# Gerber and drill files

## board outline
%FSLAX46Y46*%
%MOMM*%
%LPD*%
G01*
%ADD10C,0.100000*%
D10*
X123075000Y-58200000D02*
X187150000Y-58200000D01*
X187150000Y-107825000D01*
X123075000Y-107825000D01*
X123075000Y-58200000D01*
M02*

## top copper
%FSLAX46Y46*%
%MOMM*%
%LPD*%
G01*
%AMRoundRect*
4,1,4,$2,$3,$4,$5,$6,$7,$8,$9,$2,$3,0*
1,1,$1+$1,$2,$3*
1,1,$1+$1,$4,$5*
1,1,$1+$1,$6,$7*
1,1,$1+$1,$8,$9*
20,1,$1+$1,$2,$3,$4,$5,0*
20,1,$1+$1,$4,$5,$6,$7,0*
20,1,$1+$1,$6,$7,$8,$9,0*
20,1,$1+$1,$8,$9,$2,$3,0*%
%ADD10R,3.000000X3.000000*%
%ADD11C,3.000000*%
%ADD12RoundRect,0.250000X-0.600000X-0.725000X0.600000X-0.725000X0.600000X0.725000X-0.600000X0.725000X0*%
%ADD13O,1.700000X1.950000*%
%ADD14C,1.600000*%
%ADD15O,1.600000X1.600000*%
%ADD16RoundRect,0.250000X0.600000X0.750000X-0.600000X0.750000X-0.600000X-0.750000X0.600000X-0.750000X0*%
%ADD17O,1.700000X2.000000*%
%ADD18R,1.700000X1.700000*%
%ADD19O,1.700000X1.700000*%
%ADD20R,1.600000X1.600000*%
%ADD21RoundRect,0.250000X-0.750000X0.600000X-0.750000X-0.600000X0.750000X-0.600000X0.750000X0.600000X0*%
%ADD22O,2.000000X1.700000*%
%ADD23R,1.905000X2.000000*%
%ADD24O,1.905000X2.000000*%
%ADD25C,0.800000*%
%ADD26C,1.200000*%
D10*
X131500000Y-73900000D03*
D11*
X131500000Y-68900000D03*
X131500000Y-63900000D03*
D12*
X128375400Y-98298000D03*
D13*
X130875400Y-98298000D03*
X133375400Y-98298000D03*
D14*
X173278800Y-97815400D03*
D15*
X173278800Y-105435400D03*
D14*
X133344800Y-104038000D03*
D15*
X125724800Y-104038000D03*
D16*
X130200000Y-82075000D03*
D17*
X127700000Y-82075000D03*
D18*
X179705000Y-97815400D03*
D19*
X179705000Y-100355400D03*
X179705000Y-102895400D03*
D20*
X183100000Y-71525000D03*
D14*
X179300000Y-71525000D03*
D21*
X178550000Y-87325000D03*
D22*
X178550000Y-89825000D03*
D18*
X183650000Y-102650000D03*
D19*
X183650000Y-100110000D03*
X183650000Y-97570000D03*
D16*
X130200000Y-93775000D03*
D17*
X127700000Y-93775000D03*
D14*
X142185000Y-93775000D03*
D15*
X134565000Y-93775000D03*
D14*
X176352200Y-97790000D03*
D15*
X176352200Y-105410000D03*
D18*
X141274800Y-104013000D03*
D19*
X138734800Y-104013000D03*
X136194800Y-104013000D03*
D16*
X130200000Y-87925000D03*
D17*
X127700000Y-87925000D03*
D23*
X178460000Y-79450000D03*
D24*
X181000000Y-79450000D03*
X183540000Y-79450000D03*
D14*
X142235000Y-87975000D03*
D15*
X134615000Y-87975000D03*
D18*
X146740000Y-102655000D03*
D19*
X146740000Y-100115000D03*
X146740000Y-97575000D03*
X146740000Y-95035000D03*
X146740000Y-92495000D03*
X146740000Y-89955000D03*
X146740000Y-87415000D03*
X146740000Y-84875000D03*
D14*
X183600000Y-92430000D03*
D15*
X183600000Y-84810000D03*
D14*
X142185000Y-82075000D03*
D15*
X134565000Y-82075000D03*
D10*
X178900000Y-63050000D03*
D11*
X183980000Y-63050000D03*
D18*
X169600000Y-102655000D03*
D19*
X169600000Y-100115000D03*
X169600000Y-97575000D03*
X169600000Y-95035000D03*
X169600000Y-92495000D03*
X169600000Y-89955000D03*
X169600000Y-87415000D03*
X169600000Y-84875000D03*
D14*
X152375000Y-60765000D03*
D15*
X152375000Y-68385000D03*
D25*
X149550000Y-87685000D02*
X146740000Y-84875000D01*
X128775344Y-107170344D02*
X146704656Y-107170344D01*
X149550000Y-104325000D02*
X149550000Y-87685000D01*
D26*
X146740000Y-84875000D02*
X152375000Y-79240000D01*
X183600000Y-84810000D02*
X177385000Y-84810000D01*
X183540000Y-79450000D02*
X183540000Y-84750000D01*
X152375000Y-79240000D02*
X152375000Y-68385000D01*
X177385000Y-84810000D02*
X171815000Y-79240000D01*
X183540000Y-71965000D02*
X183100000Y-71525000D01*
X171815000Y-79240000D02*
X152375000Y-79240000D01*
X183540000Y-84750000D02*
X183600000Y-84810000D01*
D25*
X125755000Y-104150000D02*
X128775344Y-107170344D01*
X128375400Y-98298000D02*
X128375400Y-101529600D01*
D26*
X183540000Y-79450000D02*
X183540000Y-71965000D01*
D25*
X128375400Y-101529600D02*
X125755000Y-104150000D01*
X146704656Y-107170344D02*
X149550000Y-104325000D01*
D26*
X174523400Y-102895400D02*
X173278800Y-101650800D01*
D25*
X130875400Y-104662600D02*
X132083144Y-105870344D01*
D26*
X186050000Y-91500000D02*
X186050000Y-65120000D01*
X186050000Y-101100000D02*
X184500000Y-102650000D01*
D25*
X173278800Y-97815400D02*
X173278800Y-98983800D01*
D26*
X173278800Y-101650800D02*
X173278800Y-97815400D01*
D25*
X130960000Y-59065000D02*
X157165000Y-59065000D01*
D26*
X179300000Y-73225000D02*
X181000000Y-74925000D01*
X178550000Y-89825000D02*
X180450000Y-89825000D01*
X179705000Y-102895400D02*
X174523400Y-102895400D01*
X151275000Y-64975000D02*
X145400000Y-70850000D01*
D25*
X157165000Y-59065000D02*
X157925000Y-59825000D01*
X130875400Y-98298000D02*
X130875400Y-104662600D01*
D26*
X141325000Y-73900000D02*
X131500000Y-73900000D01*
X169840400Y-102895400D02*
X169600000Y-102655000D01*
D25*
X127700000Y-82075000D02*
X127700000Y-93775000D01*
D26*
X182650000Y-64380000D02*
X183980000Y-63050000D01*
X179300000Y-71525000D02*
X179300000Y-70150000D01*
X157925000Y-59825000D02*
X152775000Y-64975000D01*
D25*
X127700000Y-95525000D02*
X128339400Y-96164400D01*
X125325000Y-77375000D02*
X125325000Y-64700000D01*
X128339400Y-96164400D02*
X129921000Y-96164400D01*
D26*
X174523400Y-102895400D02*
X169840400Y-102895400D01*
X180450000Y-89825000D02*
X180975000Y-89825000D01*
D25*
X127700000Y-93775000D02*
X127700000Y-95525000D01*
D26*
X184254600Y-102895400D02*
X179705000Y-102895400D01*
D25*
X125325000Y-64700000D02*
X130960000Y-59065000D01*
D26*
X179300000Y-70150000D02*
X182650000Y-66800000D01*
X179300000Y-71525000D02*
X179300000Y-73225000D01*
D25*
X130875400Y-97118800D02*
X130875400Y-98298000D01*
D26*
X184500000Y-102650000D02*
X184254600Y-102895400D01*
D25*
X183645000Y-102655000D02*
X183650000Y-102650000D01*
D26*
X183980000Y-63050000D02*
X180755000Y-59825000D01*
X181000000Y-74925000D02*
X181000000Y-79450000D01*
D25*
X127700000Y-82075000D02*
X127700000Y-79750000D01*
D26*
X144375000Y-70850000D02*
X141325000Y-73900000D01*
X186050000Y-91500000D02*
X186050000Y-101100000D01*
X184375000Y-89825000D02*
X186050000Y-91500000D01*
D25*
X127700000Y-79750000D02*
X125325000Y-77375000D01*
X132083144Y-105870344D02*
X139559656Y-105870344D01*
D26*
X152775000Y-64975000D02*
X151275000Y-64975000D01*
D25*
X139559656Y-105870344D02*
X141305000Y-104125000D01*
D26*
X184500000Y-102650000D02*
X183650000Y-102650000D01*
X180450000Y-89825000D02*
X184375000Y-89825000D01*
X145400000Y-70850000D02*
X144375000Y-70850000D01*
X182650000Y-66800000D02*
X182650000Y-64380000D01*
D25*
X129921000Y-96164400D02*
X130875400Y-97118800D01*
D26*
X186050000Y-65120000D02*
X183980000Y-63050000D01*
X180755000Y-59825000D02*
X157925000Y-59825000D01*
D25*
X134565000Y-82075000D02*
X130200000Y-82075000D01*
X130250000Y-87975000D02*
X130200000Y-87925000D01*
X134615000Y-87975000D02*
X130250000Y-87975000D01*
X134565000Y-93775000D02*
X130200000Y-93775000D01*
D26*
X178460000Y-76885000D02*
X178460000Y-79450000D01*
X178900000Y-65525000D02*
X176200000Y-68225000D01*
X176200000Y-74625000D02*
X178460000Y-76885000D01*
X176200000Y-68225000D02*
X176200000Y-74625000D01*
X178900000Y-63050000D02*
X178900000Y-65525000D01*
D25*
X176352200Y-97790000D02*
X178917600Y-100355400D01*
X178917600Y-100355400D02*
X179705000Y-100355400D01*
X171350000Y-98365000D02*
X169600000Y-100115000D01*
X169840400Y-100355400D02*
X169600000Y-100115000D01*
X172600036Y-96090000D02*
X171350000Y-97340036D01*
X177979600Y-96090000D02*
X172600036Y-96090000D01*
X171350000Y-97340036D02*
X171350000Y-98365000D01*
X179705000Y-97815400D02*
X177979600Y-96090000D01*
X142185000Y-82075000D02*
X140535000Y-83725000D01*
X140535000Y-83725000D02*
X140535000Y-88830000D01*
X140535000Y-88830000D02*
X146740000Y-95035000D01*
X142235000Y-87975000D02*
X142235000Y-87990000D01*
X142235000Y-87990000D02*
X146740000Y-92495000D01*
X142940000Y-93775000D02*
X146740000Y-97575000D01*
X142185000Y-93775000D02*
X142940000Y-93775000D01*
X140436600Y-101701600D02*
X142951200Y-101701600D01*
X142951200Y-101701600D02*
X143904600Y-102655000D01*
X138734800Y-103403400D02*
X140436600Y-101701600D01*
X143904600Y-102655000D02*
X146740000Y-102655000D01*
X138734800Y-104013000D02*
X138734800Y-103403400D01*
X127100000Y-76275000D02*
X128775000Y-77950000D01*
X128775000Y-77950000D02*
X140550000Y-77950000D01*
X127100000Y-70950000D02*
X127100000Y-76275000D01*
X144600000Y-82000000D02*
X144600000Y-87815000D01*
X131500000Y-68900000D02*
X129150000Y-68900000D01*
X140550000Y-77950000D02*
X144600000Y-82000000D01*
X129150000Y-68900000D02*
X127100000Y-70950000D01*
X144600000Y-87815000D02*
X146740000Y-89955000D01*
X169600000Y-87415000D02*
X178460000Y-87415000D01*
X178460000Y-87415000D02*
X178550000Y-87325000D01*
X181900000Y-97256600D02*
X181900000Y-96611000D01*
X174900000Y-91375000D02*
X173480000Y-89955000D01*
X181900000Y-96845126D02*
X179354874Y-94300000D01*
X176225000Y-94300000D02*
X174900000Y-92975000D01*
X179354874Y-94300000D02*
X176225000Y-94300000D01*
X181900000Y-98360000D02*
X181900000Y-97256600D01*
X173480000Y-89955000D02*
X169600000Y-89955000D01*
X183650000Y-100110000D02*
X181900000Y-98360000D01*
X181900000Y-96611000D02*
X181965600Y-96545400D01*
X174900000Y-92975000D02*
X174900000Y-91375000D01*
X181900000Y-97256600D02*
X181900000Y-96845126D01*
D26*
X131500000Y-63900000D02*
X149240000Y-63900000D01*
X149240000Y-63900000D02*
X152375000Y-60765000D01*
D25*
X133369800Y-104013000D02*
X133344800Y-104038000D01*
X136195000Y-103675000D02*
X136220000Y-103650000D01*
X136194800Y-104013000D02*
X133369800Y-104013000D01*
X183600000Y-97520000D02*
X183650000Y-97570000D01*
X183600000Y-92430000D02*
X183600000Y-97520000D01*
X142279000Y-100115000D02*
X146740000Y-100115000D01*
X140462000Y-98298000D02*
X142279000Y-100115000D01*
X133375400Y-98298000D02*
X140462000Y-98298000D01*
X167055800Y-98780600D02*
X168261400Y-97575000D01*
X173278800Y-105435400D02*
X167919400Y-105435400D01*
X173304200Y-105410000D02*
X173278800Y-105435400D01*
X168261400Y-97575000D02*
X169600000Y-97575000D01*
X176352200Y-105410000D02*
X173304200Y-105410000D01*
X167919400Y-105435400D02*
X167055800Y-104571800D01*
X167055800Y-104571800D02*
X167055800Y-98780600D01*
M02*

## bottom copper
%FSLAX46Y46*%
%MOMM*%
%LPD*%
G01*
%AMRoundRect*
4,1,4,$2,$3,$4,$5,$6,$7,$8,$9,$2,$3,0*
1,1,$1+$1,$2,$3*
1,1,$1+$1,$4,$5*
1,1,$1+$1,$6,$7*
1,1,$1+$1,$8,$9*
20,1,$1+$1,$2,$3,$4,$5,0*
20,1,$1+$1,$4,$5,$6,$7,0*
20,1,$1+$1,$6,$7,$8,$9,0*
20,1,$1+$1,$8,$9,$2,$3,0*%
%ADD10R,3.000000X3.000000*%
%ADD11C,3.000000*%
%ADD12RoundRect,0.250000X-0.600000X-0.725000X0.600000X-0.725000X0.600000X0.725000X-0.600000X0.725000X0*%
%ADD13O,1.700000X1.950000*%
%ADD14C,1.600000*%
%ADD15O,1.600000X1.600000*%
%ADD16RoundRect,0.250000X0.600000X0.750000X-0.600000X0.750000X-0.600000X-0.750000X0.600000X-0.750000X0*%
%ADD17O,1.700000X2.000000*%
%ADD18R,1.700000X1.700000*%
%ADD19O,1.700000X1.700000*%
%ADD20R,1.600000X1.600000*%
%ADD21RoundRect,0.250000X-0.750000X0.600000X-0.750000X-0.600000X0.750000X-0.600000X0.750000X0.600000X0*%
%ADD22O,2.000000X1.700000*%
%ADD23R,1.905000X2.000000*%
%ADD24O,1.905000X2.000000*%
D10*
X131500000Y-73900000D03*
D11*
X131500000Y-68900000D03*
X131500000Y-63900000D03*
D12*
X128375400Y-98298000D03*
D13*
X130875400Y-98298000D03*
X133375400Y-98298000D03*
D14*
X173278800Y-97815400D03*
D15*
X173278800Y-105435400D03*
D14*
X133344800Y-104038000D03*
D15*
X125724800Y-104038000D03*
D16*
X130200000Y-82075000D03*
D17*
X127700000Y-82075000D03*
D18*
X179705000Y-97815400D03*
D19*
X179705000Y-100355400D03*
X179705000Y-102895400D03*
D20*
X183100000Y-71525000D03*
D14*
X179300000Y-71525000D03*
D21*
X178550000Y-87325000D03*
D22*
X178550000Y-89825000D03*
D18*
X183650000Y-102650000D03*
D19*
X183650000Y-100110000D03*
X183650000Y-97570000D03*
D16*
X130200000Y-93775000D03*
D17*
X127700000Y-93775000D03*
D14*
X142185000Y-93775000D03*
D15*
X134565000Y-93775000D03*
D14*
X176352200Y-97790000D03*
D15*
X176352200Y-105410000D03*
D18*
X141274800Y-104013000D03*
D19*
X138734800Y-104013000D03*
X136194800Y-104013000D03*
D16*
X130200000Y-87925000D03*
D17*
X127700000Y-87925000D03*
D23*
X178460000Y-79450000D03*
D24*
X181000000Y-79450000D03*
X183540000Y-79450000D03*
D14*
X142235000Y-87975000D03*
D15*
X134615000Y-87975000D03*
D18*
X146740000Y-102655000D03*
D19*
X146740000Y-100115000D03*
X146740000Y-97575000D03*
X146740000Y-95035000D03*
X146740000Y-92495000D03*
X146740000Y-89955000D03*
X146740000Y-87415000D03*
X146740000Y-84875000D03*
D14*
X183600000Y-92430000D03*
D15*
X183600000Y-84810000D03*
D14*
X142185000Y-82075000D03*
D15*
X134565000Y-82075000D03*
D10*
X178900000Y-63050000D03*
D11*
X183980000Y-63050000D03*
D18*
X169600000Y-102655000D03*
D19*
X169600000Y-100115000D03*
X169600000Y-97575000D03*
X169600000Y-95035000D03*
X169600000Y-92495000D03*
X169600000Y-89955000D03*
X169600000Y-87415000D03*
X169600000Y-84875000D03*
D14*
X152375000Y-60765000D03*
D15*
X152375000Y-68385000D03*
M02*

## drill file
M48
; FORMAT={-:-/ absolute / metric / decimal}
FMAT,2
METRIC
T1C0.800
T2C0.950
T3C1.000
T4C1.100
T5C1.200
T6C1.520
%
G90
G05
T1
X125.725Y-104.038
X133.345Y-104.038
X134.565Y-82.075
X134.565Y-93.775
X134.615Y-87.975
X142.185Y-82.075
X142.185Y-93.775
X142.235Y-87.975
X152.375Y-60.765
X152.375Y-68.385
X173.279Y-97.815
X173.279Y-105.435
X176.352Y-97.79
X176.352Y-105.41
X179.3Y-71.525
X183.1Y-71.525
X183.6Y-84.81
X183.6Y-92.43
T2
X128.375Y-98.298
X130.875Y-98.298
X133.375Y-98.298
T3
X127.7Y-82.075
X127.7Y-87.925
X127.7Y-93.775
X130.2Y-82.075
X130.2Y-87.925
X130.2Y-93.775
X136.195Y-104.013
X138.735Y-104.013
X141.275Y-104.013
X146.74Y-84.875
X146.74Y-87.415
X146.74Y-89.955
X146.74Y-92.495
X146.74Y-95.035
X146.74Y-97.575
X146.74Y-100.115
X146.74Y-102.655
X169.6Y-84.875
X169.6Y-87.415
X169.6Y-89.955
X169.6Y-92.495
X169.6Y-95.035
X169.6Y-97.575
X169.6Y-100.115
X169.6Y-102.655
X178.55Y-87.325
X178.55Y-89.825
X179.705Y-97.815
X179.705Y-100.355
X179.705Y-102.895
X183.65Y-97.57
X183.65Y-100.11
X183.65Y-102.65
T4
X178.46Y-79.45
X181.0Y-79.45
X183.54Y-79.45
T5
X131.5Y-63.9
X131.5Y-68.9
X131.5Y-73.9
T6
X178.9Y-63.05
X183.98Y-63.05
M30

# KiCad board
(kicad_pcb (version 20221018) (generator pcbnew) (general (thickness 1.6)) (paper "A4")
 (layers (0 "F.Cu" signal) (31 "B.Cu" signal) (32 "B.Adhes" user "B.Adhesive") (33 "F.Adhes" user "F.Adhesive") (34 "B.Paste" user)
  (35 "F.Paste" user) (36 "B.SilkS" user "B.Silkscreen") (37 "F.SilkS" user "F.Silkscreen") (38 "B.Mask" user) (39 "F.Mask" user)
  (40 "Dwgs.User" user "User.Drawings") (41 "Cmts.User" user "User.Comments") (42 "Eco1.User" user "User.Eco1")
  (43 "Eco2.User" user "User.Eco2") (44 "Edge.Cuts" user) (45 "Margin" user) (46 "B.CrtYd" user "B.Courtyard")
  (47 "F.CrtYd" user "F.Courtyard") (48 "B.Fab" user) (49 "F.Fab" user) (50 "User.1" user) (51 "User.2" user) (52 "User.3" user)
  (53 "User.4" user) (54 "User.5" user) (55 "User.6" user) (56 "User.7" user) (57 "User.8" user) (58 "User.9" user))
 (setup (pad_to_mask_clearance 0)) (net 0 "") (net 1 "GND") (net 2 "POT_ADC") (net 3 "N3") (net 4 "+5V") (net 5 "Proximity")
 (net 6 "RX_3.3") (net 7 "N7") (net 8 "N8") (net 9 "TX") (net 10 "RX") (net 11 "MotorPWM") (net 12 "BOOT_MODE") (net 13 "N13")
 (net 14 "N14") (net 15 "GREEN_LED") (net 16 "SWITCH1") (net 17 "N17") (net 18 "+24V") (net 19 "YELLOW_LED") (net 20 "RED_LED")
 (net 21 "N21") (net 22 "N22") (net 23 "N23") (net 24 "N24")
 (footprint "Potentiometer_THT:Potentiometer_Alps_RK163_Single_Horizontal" (layer "F.Cu") (at 131.5 73.9 180)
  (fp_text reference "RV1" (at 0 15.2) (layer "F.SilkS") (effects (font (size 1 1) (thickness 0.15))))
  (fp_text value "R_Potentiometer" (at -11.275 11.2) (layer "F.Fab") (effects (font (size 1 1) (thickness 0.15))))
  (pad "1" thru_hole rect (at 0 0) (size 3 3) (drill 1.2) (layers "*.Cu" "*.Mask") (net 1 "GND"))
  (pad "2" thru_hole circle (at 0 5) (size 3 3) (drill 1.2) (layers "*.Cu" "*.Mask") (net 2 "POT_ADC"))
  (pad "3" thru_hole circle (at 0 10) (size 3 3) (drill 1.2) (layers "*.Cu" "*.Mask") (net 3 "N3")))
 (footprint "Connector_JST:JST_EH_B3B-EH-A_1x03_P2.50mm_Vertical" (layer "F.Cu") (at 128.3754 98.298)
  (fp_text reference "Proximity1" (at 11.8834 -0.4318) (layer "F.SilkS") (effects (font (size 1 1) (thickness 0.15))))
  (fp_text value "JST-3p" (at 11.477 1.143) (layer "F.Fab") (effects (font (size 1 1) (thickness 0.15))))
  (pad "1" thru_hole roundrect (at 0 0) (size 1.7 1.95) (drill 0.95) (layers "*.Cu" "*.Mask") (roundrect_rratio 0.147059) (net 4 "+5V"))
  (pad "2" thru_hole oval (at 2.5 0) (size 1.7 1.95) (drill 0.95) (layers "*.Cu" "*.Mask") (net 1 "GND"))
  (pad "3" thru_hole oval (at 5 0) (size 1.7 1.95) (drill 0.95) (layers "*.Cu" "*.Mask") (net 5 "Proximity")))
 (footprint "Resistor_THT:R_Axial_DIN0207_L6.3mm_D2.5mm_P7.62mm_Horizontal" (layer "F.Cu") (at 173.2788 97.8154 -90)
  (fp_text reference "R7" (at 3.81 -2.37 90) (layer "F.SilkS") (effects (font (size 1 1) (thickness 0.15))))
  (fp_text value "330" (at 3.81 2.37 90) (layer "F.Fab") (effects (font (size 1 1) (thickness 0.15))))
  (pad "1" thru_hole circle (at 0 0 270) (size 1.6 1.6) (drill 0.8) (layers "*.Cu" "*.Mask") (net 1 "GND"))
  (pad "2" thru_hole oval (at 7.62 0 270) (size 1.6 1.6) (drill 0.8) (layers "*.Cu" "*.Mask") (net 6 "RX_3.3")))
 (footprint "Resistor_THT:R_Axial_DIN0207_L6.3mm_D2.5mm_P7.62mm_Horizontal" (layer "F.Cu") (at 133.3448 104.038 180)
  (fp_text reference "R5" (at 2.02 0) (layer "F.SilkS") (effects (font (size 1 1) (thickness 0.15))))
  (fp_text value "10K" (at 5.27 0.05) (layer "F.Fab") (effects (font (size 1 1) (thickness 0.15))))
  (pad "1" thru_hole circle (at 0 0 180) (size 1.6 1.6) (drill 0.8) (layers "*.Cu" "*.Mask") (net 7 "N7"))
  (pad "2" thru_hole oval (at 7.62 0 180) (size 1.6 1.6) (drill 0.8) (layers "*.Cu" "*.Mask") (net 4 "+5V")))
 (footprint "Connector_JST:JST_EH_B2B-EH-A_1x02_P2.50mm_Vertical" (layer "F.Cu") (at 130.2 82.075 180)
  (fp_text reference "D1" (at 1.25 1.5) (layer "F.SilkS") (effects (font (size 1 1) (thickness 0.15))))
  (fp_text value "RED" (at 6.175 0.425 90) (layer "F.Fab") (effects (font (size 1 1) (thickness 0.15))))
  (pad "1" thru_hole roundrect (at 0 0 180) (size 1.7 2) (drill 1) (layers "*.Cu" "*.Mask") (roundrect_rratio 0.147059) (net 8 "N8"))
  (pad "2" thru_hole oval (at 2.5 0 180) (size 1.7 2) (drill 1) (layers "*.Cu" "*.Mask") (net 1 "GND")))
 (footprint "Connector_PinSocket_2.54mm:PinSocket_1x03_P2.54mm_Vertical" (layer "F.Cu") (at 179.705 97.8154)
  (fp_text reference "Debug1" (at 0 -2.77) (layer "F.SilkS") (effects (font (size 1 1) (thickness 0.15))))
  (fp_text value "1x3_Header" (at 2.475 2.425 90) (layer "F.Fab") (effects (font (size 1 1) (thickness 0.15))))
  (pad "1" thru_hole rect (at 0 0) (size 1.7 1.7) (drill 1) (layers "*.Cu" "*.Mask") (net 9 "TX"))
  (pad "2" thru_hole oval (at 0 2.54) (size 1.7 1.7) (drill 1) (layers "*.Cu" "*.Mask") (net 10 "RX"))
  (pad "3" thru_hole oval (at 0 5.08) (size 1.7 1.7) (drill 1) (layers "*.Cu" "*.Mask") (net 1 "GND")))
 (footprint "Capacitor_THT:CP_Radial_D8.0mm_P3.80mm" (layer "F.Cu") (at 183.1 71.525 180)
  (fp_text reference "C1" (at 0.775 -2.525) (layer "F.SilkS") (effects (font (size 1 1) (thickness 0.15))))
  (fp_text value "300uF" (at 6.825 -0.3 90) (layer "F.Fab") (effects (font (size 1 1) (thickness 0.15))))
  (pad "1" thru_hole rect (at 0 0 180) (size 1.6 1.6) (drill 0.8) (layers "*.Cu" "*.Mask") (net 4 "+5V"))
  (pad "2" thru_hole circle (at 3.8 0 180) (size 1.6 1.6) (drill 0.8) (layers "*.Cu" "*.Mask") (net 1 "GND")))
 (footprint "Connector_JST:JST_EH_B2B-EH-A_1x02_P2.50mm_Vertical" (layer "F.Cu") (at 178.55 87.325 -90)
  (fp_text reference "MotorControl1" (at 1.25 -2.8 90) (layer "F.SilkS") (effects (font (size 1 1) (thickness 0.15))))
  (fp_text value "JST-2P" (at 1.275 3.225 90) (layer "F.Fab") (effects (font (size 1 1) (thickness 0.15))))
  (pad "1" thru_hole roundrect (at 0 0 270) (size 1.7 2) (drill 1) (layers "*.Cu" "*.Mask") (roundrect_rratio 0.147059) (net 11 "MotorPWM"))
  (pad "2" thru_hole oval (at 2.5 0 270) (size 1.7 2) (drill 1) (layers "*.Cu" "*.Mask") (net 1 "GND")))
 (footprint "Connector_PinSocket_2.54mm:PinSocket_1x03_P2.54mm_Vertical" (layer "F.Cu") (at 183.65 102.65 180)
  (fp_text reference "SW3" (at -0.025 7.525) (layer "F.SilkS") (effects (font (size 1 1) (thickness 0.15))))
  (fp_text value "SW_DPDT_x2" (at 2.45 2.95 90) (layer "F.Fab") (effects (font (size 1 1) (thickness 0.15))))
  (pad "1" thru_hole rect (at 0 0 180) (size 1.7 1.7) (drill 1) (layers "*.Cu" "*.Mask") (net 1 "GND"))
  (pad "2" thru_hole oval (at 0 2.54 180) (size 1.7 1.7) (drill 1) (layers "*.Cu" "*.Mask") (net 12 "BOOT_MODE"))
  (pad "3" thru_hole oval (at 0 5.08 180) (size 1.7 1.7) (drill 1) (layers "*.Cu" "*.Mask") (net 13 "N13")))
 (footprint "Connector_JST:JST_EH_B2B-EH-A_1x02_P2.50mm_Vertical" (layer "F.Cu") (at 130.2 93.775 180)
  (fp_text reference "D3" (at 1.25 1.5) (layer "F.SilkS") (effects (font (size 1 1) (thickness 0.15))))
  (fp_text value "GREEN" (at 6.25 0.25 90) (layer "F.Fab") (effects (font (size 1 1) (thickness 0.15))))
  (pad "1" thru_hole roundrect (at 0 0 180) (size 1.7 2) (drill 1) (layers "*.Cu" "*.Mask") (roundrect_rratio 0.147059) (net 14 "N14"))
  (pad "2" thru_hole oval (at 2.5 0 180) (size 1.7 2) (drill 1) (layers "*.Cu" "*.Mask") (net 1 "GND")))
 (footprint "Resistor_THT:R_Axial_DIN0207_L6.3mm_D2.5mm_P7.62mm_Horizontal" (layer "F.Cu") (at 142.185 93.775 180)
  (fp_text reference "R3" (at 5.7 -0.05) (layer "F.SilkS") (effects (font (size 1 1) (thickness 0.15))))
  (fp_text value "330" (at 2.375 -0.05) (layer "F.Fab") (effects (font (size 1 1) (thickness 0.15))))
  (pad "1" thru_hole circle (at 0 0 180) (size 1.6 1.6) (drill 0.8) (layers "*.Cu" "*.Mask") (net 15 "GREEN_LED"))
  (pad "2" thru_hole oval (at 7.62 0 180) (size 1.6 1.6) (drill 0.8) (layers "*.Cu" "*.Mask") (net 14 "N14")))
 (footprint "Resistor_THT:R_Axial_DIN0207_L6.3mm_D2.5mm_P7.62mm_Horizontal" (layer "F.Cu") (at 176.3522 97.79 -90)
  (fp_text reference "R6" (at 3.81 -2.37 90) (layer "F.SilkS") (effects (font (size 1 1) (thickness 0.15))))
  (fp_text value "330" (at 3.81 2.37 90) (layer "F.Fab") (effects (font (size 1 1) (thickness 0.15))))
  (pad "1" thru_hole circle (at 0 0 270) (size 1.6 1.6) (drill 0.8) (layers "*.Cu" "*.Mask") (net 10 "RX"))
  (pad "2" thru_hole oval (at 7.62 0 270) (size 1.6 1.6) (drill 0.8) (layers "*.Cu" "*.Mask") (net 6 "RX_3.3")))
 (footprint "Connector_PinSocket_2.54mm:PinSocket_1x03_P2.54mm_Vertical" (layer "F.Cu") (at 141.2748 104.013 -90)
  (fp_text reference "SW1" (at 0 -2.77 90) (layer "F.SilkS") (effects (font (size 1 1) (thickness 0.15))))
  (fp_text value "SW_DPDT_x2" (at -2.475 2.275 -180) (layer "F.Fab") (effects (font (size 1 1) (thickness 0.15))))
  (pad "1" thru_hole rect (at 0 0 270) (size 1.7 1.7) (drill 1) (layers "*.Cu" "*.Mask") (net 1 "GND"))
  (pad "2" thru_hole oval (at 0 2.54 270) (size 1.7 1.7) (drill 1) (layers "*.Cu" "*.Mask") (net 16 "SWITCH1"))
  (pad "3" thru_hole oval (at 0 5.08 270) (size 1.7 1.7) (drill 1) (layers "*.Cu" "*.Mask") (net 7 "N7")))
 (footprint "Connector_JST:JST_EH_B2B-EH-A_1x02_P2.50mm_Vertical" (layer "F.Cu") (at 130.2 87.925 180)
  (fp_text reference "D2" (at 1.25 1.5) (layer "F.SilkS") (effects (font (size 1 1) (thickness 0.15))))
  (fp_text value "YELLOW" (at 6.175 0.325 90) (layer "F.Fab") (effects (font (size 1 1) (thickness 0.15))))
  (pad "1" thru_hole roundrect (at 0 0 180) (size 1.7 2) (drill 1) (layers "*.Cu" "*.Mask") (roundrect_rratio 0.147059) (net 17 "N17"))
  (pad "2" thru_hole oval (at 2.5 0 180) (size 1.7 2) (drill 1) (layers "*.Cu" "*.Mask") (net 1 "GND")))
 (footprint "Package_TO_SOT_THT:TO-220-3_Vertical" (layer "F.Cu") (at 178.46 79.45)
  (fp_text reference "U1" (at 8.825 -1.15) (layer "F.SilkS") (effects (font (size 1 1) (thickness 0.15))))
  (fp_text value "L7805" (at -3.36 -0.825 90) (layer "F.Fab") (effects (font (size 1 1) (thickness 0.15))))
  (pad "1" thru_hole rect (at 0 0) (size 1.905 2) (drill 1.1) (layers "*.Cu" "*.Mask") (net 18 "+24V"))
  (pad "2" thru_hole oval (at 2.54 0) (size 1.905 2) (drill 1.1) (layers "*.Cu" "*.Mask") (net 1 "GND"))
  (pad "3" thru_hole oval (at 5.08 0) (size 1.905 2) (drill 1.1) (layers "*.Cu" "*.Mask") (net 4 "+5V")))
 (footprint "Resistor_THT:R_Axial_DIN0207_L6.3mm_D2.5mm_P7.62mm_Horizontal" (layer "F.Cu") (at 142.235 87.975 180)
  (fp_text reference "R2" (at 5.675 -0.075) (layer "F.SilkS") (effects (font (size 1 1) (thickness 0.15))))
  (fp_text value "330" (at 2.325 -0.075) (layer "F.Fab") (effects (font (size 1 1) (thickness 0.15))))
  (pad "1" thru_hole circle (at 0 0 180) (size 1.6 1.6) (drill 0.8) (layers "*.Cu" "*.Mask") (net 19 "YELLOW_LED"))
  (pad "2" thru_hole oval (at 7.62 0 180) (size 1.6 1.6) (drill 0.8) (layers "*.Cu" "*.Mask") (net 17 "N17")))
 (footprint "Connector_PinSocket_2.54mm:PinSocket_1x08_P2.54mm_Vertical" (layer "F.Cu") (at 146.74 102.655 180)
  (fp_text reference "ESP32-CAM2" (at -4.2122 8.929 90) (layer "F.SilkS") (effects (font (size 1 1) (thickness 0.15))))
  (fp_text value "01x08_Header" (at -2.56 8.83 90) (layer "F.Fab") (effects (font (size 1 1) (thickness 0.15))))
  (pad "1" thru_hole rect (at 0 0 180) (size 1.7 1.7) (drill 1) (layers "*.Cu" "*.Mask") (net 16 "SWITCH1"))
  (pad "2" thru_hole oval (at 0 2.54 180) (size 1.7 1.7) (drill 1) (layers "*.Cu" "*.Mask") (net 5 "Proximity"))
  (pad "3" thru_hole oval (at 0 5.08 180) (size 1.7 1.7) (drill 1) (layers "*.Cu" "*.Mask") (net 15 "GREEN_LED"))
  (pad "4" thru_hole oval (at 0 7.62 180) (size 1.7 1.7) (drill 1) (layers "*.Cu" "*.Mask") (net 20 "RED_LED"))
  (pad "5" thru_hole oval (at 0 10.16 180) (size 1.7 1.7) (drill 1) (layers "*.Cu" "*.Mask") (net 19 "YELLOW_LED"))
  (pad "6" thru_hole oval (at 0 12.7 180) (size 1.7 1.7) (drill 1) (layers "*.Cu" "*.Mask") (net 2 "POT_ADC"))
  (pad "7" thru_hole oval (at 0 15.24 180) (size 1.7 1.7) (drill 1) (layers "*.Cu" "*.Mask") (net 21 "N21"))
  (pad "8" thru_hole oval (at 0 17.78 180) (size 1.7 1.7) (drill 1) (layers "*.Cu" "*.Mask") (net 4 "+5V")))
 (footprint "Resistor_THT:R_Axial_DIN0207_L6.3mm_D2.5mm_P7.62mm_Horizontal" (layer "F.Cu") (at 183.6 92.43 90)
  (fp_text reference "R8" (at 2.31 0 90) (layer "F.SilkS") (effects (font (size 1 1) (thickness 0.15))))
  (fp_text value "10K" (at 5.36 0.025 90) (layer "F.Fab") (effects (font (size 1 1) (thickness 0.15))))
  (pad "1" thru_hole circle (at 0 0 90) (size 1.6 1.6) (drill 0.8) (layers "*.Cu" "*.Mask") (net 13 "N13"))
  (pad "2" thru_hole oval (at 7.62 0 90) (size 1.6 1.6) (drill 0.8) (layers "*.Cu" "*.Mask") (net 4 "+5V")))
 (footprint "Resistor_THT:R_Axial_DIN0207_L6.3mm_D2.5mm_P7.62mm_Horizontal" (layer "F.Cu") (at 142.185 82.075 180)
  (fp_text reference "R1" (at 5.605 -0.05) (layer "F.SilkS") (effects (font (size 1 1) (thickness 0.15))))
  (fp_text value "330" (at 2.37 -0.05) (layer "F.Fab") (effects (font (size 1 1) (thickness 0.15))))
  (pad "1" thru_hole circle (at 0 0 180) (size 1.6 1.6) (drill 0.8) (layers "*.Cu" "*.Mask") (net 20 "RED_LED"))
  (pad "2" thru_hole oval (at 7.62 0 180) (size 1.6 1.6) (drill 0.8) (layers "*.Cu" "*.Mask") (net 8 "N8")))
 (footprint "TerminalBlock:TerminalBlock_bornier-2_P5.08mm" (layer "F.Cu") (at 178.9 63.05)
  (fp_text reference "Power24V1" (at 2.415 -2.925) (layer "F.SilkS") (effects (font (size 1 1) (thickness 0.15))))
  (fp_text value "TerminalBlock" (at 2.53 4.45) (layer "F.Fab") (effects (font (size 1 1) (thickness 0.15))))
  (pad "1" thru_hole rect (at 0 0) (size 3 3) (drill 1.52) (layers "*.Cu" "*.Mask") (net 18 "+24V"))
  (pad "2" thru_hole circle (at 5.08 0) (size 3 3) (drill 1.52) (layers "*.Cu" "*.Mask") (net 1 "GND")))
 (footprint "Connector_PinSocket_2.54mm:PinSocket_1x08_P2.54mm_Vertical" (layer "F.Cu") (at 169.6 102.655 180)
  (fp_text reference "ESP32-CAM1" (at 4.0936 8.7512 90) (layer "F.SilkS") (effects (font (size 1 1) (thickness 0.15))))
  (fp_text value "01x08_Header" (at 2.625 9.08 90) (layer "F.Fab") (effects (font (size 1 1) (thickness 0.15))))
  (pad "1" thru_hole rect (at 0 0 180) (size 1.7 1.7) (drill 1) (layers "*.Cu" "*.Mask") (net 1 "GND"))
  (pad "2" thru_hole oval (at 0 2.54 180) (size 1.7 1.7) (drill 1) (layers "*.Cu" "*.Mask") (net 9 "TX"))
  (pad "3" thru_hole oval (at 0 5.08 180) (size 1.7 1.7) (drill 1) (layers "*.Cu" "*.Mask") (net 6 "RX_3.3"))
  (pad "4" thru_hole oval (at 0 7.62 180) (size 1.7 1.7) (drill 1) (layers "*.Cu" "*.Mask") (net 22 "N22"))
  (pad "5" thru_hole oval (at 0 10.16 180) (size 1.7 1.7) (drill 1) (layers "*.Cu" "*.Mask") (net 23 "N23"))
  (pad "6" thru_hole oval (at 0 12.7 180) (size 1.7 1.7) (drill 1) (layers "*.Cu" "*.Mask") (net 12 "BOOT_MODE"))
  (pad "7" thru_hole oval (at 0 15.24 180) (size 1.7 1.7) (drill 1) (layers "*.Cu" "*.Mask") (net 11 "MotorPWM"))
  (pad "8" thru_hole oval (at 0 17.78 180) (size 1.7 1.7) (drill 1) (layers "*.Cu" "*.Mask") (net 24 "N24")))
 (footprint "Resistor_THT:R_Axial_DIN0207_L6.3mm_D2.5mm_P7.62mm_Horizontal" (layer "F.Cu") (at 152.375 60.765 -90)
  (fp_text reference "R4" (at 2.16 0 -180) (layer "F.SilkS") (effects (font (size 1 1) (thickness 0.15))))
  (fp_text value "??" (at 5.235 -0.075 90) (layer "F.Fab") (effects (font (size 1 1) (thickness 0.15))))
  (pad "1" thru_hole circle (at 0 0 270) (size 1.6 1.6) (drill 0.8) (layers "*.Cu" "*.Mask") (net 3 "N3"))
  (pad "2" thru_hole oval (at 7.62 0 270) (size 1.6 1.6) (drill 0.8) (layers "*.Cu" "*.Mask") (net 4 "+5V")))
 (gr_rect (start 123.075 58.2) (end 187.15 107.825) (stroke (width 0.1) (type default)) (fill none) (layer "Edge.Cuts"))
 (segment (start 149.55 87.685) (end 146.74 84.875) (width 0.8) (layer "F.Cu") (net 4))
 (segment (start 128.775344 107.170344) (end 146.704656 107.170344) (width 0.8) (layer "F.Cu") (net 4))
 (segment (start 149.55 104.325) (end 149.55 87.685) (width 0.8) (layer "F.Cu") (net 4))
 (segment (start 146.74 84.875) (end 152.375 79.24) (width 1.2) (layer "F.Cu") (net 4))
 (segment (start 183.6 84.81) (end 177.385 84.81) (width 1.2) (layer "F.Cu") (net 4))
 (segment (start 183.54 79.45) (end 183.54 84.75) (width 1.2) (layer "F.Cu") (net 4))
 (segment (start 152.375 79.24) (end 152.375 68.385) (width 1.2) (layer "F.Cu") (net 4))
 (segment (start 177.385 84.81) (end 171.815 79.24) (width 1.2) (layer "F.Cu") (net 4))
 (segment (start 183.54 71.965) (end 183.1 71.525) (width 1.2) (layer "F.Cu") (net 4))
 (segment (start 171.815 79.24) (end 152.375 79.24) (width 1.2) (layer "F.Cu") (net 4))
 (segment (start 183.54 84.75) (end 183.6 84.81) (width 1.2) (layer "F.Cu") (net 4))
 (segment (start 125.755 104.15) (end 128.775344 107.170344) (width 0.8) (layer "F.Cu") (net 4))
 (segment (start 128.3754 98.298) (end 128.3754 101.5296) (width 0.8) (layer "F.Cu") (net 4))
 (segment (start 183.54 79.45) (end 183.54 71.965) (width 1.2) (layer "F.Cu") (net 4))
 (segment (start 128.3754 101.5296) (end 125.755 104.15) (width 0.8) (layer "F.Cu") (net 4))
 (segment (start 146.704656 107.170344) (end 149.55 104.325) (width 0.8) (layer "F.Cu") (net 4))
 (segment (start 174.5234 102.8954) (end 173.2788 101.6508) (width 1.2) (layer "F.Cu") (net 1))
 (segment (start 130.8754 104.6626) (end 132.083144 105.870344) (width 0.8) (layer "F.Cu") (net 1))
 (segment (start 186.05 91.5) (end 186.05 65.12) (width 1.2) (layer "F.Cu") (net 1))
 (segment (start 186.05 101.1) (end 184.5 102.65) (width 1.2) (layer "F.Cu") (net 1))
 (segment (start 173.2788 97.8154) (end 173.2788 98.9838) (width 0.8) (layer "F.Cu") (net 1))
 (segment (start 173.2788 101.6508) (end 173.2788 97.8154) (width 1.2) (layer "F.Cu") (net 1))
 (segment (start 130.96 59.065) (end 157.165 59.065) (width 0.8) (layer "F.Cu") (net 1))
 (segment (start 179.3 73.225) (end 181 74.925) (width 1.2) (layer "F.Cu") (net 1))
 (segment (start 178.55 89.825) (end 180.45 89.825) (width 1.2) (layer "F.Cu") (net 1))
 (segment (start 179.705 102.8954) (end 174.5234 102.8954) (width 1.2) (layer "F.Cu") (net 1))
 (segment (start 151.275 64.975) (end 145.4 70.85) (width 1.2) (layer "F.Cu") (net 1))
 (segment (start 157.165 59.065) (end 157.925 59.825) (width 0.8) (layer "F.Cu") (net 1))
 (segment (start 130.8754 98.298) (end 130.8754 104.6626) (width 0.8) (layer "F.Cu") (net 1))
 (segment (start 141.325 73.9) (end 131.5 73.9) (width 1.2) (layer "F.Cu") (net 1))
 (segment (start 169.8404 102.8954) (end 169.6 102.655) (width 1.2) (layer "F.Cu") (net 1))
 (segment (start 127.7 82.075) (end 127.7 93.775) (width 0.8) (layer "F.Cu") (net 1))
 (segment (start 182.65 64.38) (end 183.98 63.05) (width 1.2) (layer "F.Cu") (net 1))
 (segment (start 179.3 71.525) (end 179.3 70.15) (width 1.2) (layer "F.Cu") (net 1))
 (segment (start 157.925 59.825) (end 152.775 64.975) (width 1.2) (layer "F.Cu") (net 1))
 (segment (start 127.7 95.525) (end 128.3394 96.1644) (width 0.8) (layer "F.Cu") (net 1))
 (segment (start 125.325 77.375) (end 125.325 64.7) (width 0.8) (layer "F.Cu") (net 1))
 (segment (start 128.3394 96.1644) (end 129.921 96.1644) (width 0.8) (layer "F.Cu") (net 1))
 (segment (start 174.5234 102.8954) (end 169.8404 102.8954) (width 1.2) (layer "F.Cu") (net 1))
 (segment (start 180.45 89.825) (end 180.975 89.825) (width 1.2) (layer "F.Cu") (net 1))
 (segment (start 127.7 93.775) (end 127.7 95.525) (width 0.8) (layer "F.Cu") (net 1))
 (segment (start 184.2546 102.8954) (end 179.705 102.8954) (width 1.2) (layer "F.Cu") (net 1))
 (segment (start 125.325 64.7) (end 130.96 59.065) (width 0.8) (layer "F.Cu") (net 1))
 (segment (start 179.3 70.15) (end 182.65 66.8) (width 1.2) (layer "F.Cu") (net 1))
 (segment (start 179.3 71.525) (end 179.3 73.225) (width 1.2) (layer "F.Cu") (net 1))
 (segment (start 130.8754 97.1188) (end 130.8754 98.298) (width 0.8) (layer "F.Cu") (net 1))
 (segment (start 184.5 102.65) (end 184.2546 102.8954) (width 1.2) (layer "F.Cu") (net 1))
 (segment (start 183.645 102.655) (end 183.65 102.65) (width 0.8) (layer "F.Cu") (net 1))
 (segment (start 183.98 63.05) (end 180.755 59.825) (width 1.2) (layer "F.Cu") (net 1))
 (segment (start 181 74.925) (end 181 79.45) (width 1.2) (layer "F.Cu") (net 1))
 (segment (start 127.7 82.075) (end 127.7 79.75) (width 0.8) (layer "F.Cu") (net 1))
 (segment (start 144.375 70.85) (end 141.325 73.9) (width 1.2) (layer "F.Cu") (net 1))
 (segment (start 186.05 91.5) (end 186.05 101.1) (width 1.2) (layer "F.Cu") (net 1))
 (segment (start 184.375 89.825) (end 186.05 91.5) (width 1.2) (layer "F.Cu") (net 1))
 (segment (start 127.7 79.75) (end 125.325 77.375) (width 0.8) (layer "F.Cu") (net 1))
 (segment (start 132.083144 105.870344) (end 139.559656 105.870344) (width 0.8) (layer "F.Cu") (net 1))
 (segment (start 152.775 64.975) (end 151.275 64.975) (width 1.2) (layer "F.Cu") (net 1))
 (segment (start 139.559656 105.870344) (end 141.305 104.125) (width 0.8) (layer "F.Cu") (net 1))
 (segment (start 184.5 102.65) (end 183.65 102.65) (width 1.2) (layer "F.Cu") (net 1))
 (segment (start 180.45 89.825) (end 184.375 89.825) (width 1.2) (layer "F.Cu") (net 1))
 (segment (start 145.4 70.85) (end 144.375 70.85) (width 1.2) (layer "F.Cu") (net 1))
 (segment (start 182.65 66.8) (end 182.65 64.38) (width 1.2) (layer "F.Cu") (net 1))
 (segment (start 129.921 96.1644) (end 130.8754 97.1188) (width 0.8) (layer "F.Cu") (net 1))
 (segment (start 186.05 65.12) (end 183.98 63.05) (width 1.2) (layer "F.Cu") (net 1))
 (segment (start 180.755 59.825) (end 157.925 59.825) (width 1.2) (layer "F.Cu") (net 1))
 (segment (start 134.565 82.075) (end 130.2 82.075) (width 0.8) (layer "F.Cu") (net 8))
 (segment (start 130.25 87.975) (end 130.2 87.925) (width 0.8) (layer "F.Cu") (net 17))
 (segment (start 134.615 87.975) (end 130.25 87.975) (width 0.8) (layer "F.Cu") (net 17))
 (segment (start 134.565 93.775) (end 130.2 93.775) (width 0.8) (layer "F.Cu") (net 14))
 (segment (start 178.46 76.885) (end 178.46 79.45) (width 1.2) (layer "F.Cu") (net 18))
 (segment (start 178.9 65.525) (end 176.2 68.225) (width 1.2) (layer "F.Cu") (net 18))
 (segment (start 176.2 74.625) (end 178.46 76.885) (width 1.2) (layer "F.Cu") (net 18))
 (segment (start 176.2 68.225) (end 176.2 74.625) (width 1.2) (layer "F.Cu") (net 18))
 (segment (start 178.9 63.05) (end 178.9 65.525) (width 1.2) (layer "F.Cu") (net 18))
 (segment (start 176.3522 97.79) (end 178.9176 100.3554) (width 0.8) (layer "F.Cu") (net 10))
 (segment (start 178.9176 100.3554) (end 179.705 100.3554) (width 0.8) (layer "F.Cu") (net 10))
 (segment (start 171.35 98.365) (end 169.6 100.115) (width 0.8) (layer "F.Cu") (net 9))
 (segment (start 169.8404 100.3554) (end 169.6 100.115) (width 0.8) (layer "F.Cu") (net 9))
 (segment (start 172.600036 96.09) (end 171.35 97.340036) (width 0.8) (layer "F.Cu") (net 9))
 (segment (start 177.9796 96.09) (end 172.600036 96.09) (width 0.8) (layer "F.Cu") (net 9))
 (segment (start 171.35 97.340036) (end 171.35 98.365) (width 0.8) (layer "F.Cu") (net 9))
 (segment (start 179.705 97.8154) (end 177.9796 96.09) (width 0.8) (layer "F.Cu") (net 9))
 (segment (start 142.185 82.075) (end 140.535 83.725) (width 0.8) (layer "F.Cu") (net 20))
 (segment (start 140.535 83.725) (end 140.535 88.83) (width 0.8) (layer "F.Cu") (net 20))
 (segment (start 140.535 88.83) (end 146.74 95.035) (width 0.8) (layer "F.Cu") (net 20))
 (segment (start 142.235 87.975) (end 142.235 87.99) (width 0.8) (layer "F.Cu") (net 19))
 (segment (start 142.235 87.99) (end 146.74 92.495) (width 0.8) (layer "F.Cu") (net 19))
 (segment (start 142.94 93.775) (end 146.74 97.575) (width 0.8) (layer "F.Cu") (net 15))
 (segment (start 142.185 93.775) (end 142.94 93.775) (width 0.8) (layer "F.Cu") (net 15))
 (segment (start 140.4366 101.7016) (end 142.9512 101.7016) (width 0.8) (layer "F.Cu") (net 16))
 (segment (start 142.9512 101.7016) (end 143.9046 102.655) (width 0.8) (layer "F.Cu") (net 16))
 (segment (start 138.7348 103.4034) (end 140.4366 101.7016) (width 0.8) (layer "F.Cu") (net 16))
 (segment (start 143.9046 102.655) (end 146.74 102.655) (width 0.8) (layer "F.Cu") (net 16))
 (segment (start 138.7348 104.013) (end 138.7348 103.4034) (width 0.8) (layer "F.Cu") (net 16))
 (segment (start 127.1 76.275) (end 128.775 77.95) (width 0.8) (layer "F.Cu") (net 2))
 (segment (start 128.775 77.95) (end 140.55 77.95) (width 0.8) (layer "F.Cu") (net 2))
 (segment (start 127.1 70.95) (end 127.1 76.275) (width 0.8) (layer "F.Cu") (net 2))
 (segment (start 144.6 82) (end 144.6 87.815) (width 0.8) (layer "F.Cu") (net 2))
 (segment (start 131.5 68.9) (end 129.15 68.9) (width 0.8) (layer "F.Cu") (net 2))
 (segment (start 140.55 77.95) (end 144.6 82) (width 0.8) (layer "F.Cu") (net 2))
 (segment (start 129.15 68.9) (end 127.1 70.95) (width 0.8) (layer "F.Cu") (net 2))
 (segment (start 144.6 87.815) (end 146.74 89.955) (width 0.8) (layer "F.Cu") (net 2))
 (segment (start 169.6 87.415) (end 178.46 87.415) (width 0.8) (layer "F.Cu") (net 11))
 (segment (start 178.46 87.415) (end 178.55 87.325) (width 0.8) (layer "F.Cu") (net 11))
 (segment (start 181.9 97.2566) (end 181.9 96.611) (width 0.8) (layer "F.Cu") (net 12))
 (segment (start 174.9 91.375) (end 173.48 89.955) (width 0.8) (layer "F.Cu") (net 12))
 (segment (start 181.9 96.845126) (end 179.354874 94.3) (width 0.8) (layer "F.Cu") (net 12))
 (segment (start 176.225 94.3) (end 174.9 92.975) (width 0.8) (layer "F.Cu") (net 12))
 (segment (start 179.354874 94.3) (end 176.225 94.3) (width 0.8) (layer "F.Cu") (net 12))
 (segment (start 181.9 98.36) (end 181.9 97.2566) (width 0.8) (layer "F.Cu") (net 12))
 (segment (start 173.48 89.955) (end 169.6 89.955) (width 0.8) (layer "F.Cu") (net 12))
 (segment (start 183.65 100.11) (end 181.9 98.36) (width 0.8) (layer "F.Cu") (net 12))
 (segment (start 181.9 96.611) (end 181.9656 96.5454) (width 0.8) (layer "F.Cu") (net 12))
 (segment (start 174.9 92.975) (end 174.9 91.375) (width 0.8) (layer "F.Cu") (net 12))
 (segment (start 181.9 97.2566) (end 181.9 96.845126) (width 0.8) (layer "F.Cu") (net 12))
 (segment (start 131.5 63.9) (end 149.24 63.9) (width 1.2) (layer "F.Cu") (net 3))
 (segment (start 149.24 63.9) (end 152.375 60.765) (width 1.2) (layer "F.Cu") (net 3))
 (segment (start 133.3698 104.013) (end 133.3448 104.038) (width 0.8) (layer "F.Cu") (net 7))
 (segment (start 136.195 103.675) (end 136.22 103.65) (width 0.8) (layer "F.Cu") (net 7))
 (segment (start 136.1948 104.013) (end 133.3698 104.013) (width 0.8) (layer "F.Cu") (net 7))
 (segment (start 183.6 97.52) (end 183.65 97.57) (width 0.8) (layer "F.Cu") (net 13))
 (segment (start 183.6 92.43) (end 183.6 97.52) (width 0.8) (layer "F.Cu") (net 13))
 (segment (start 142.279 100.115) (end 146.74 100.115) (width 0.8) (layer "F.Cu") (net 5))
 (segment (start 140.462 98.298) (end 142.279 100.115) (width 0.8) (layer "F.Cu") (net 5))
 (segment (start 133.3754 98.298) (end 140.462 98.298) (width 0.8) (layer "F.Cu") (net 5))
 (segment (start 167.0558 98.7806) (end 168.2614 97.575) (width 0.8) (layer "F.Cu") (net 6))
 (segment (start 173.2788 105.4354) (end 167.9194 105.4354) (width 0.8) (layer "F.Cu") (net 6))
 (segment (start 173.3042 105.41) (end 173.2788 105.4354) (width 0.8) (layer "F.Cu") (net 6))
 (segment (start 168.2614 97.575) (end 169.6 97.575) (width 0.8) (layer "F.Cu") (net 6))
 (segment (start 176.3522 105.41) (end 173.3042 105.41) (width 0.8) (layer "F.Cu") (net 6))
 (segment (start 167.9194 105.4354) (end 167.0558 104.5718) (width 0.8) (layer "F.Cu") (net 6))
 (segment (start 167.0558 104.5718) (end 167.0558 98.7806) (width 0.8) (layer "F.Cu") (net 6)))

